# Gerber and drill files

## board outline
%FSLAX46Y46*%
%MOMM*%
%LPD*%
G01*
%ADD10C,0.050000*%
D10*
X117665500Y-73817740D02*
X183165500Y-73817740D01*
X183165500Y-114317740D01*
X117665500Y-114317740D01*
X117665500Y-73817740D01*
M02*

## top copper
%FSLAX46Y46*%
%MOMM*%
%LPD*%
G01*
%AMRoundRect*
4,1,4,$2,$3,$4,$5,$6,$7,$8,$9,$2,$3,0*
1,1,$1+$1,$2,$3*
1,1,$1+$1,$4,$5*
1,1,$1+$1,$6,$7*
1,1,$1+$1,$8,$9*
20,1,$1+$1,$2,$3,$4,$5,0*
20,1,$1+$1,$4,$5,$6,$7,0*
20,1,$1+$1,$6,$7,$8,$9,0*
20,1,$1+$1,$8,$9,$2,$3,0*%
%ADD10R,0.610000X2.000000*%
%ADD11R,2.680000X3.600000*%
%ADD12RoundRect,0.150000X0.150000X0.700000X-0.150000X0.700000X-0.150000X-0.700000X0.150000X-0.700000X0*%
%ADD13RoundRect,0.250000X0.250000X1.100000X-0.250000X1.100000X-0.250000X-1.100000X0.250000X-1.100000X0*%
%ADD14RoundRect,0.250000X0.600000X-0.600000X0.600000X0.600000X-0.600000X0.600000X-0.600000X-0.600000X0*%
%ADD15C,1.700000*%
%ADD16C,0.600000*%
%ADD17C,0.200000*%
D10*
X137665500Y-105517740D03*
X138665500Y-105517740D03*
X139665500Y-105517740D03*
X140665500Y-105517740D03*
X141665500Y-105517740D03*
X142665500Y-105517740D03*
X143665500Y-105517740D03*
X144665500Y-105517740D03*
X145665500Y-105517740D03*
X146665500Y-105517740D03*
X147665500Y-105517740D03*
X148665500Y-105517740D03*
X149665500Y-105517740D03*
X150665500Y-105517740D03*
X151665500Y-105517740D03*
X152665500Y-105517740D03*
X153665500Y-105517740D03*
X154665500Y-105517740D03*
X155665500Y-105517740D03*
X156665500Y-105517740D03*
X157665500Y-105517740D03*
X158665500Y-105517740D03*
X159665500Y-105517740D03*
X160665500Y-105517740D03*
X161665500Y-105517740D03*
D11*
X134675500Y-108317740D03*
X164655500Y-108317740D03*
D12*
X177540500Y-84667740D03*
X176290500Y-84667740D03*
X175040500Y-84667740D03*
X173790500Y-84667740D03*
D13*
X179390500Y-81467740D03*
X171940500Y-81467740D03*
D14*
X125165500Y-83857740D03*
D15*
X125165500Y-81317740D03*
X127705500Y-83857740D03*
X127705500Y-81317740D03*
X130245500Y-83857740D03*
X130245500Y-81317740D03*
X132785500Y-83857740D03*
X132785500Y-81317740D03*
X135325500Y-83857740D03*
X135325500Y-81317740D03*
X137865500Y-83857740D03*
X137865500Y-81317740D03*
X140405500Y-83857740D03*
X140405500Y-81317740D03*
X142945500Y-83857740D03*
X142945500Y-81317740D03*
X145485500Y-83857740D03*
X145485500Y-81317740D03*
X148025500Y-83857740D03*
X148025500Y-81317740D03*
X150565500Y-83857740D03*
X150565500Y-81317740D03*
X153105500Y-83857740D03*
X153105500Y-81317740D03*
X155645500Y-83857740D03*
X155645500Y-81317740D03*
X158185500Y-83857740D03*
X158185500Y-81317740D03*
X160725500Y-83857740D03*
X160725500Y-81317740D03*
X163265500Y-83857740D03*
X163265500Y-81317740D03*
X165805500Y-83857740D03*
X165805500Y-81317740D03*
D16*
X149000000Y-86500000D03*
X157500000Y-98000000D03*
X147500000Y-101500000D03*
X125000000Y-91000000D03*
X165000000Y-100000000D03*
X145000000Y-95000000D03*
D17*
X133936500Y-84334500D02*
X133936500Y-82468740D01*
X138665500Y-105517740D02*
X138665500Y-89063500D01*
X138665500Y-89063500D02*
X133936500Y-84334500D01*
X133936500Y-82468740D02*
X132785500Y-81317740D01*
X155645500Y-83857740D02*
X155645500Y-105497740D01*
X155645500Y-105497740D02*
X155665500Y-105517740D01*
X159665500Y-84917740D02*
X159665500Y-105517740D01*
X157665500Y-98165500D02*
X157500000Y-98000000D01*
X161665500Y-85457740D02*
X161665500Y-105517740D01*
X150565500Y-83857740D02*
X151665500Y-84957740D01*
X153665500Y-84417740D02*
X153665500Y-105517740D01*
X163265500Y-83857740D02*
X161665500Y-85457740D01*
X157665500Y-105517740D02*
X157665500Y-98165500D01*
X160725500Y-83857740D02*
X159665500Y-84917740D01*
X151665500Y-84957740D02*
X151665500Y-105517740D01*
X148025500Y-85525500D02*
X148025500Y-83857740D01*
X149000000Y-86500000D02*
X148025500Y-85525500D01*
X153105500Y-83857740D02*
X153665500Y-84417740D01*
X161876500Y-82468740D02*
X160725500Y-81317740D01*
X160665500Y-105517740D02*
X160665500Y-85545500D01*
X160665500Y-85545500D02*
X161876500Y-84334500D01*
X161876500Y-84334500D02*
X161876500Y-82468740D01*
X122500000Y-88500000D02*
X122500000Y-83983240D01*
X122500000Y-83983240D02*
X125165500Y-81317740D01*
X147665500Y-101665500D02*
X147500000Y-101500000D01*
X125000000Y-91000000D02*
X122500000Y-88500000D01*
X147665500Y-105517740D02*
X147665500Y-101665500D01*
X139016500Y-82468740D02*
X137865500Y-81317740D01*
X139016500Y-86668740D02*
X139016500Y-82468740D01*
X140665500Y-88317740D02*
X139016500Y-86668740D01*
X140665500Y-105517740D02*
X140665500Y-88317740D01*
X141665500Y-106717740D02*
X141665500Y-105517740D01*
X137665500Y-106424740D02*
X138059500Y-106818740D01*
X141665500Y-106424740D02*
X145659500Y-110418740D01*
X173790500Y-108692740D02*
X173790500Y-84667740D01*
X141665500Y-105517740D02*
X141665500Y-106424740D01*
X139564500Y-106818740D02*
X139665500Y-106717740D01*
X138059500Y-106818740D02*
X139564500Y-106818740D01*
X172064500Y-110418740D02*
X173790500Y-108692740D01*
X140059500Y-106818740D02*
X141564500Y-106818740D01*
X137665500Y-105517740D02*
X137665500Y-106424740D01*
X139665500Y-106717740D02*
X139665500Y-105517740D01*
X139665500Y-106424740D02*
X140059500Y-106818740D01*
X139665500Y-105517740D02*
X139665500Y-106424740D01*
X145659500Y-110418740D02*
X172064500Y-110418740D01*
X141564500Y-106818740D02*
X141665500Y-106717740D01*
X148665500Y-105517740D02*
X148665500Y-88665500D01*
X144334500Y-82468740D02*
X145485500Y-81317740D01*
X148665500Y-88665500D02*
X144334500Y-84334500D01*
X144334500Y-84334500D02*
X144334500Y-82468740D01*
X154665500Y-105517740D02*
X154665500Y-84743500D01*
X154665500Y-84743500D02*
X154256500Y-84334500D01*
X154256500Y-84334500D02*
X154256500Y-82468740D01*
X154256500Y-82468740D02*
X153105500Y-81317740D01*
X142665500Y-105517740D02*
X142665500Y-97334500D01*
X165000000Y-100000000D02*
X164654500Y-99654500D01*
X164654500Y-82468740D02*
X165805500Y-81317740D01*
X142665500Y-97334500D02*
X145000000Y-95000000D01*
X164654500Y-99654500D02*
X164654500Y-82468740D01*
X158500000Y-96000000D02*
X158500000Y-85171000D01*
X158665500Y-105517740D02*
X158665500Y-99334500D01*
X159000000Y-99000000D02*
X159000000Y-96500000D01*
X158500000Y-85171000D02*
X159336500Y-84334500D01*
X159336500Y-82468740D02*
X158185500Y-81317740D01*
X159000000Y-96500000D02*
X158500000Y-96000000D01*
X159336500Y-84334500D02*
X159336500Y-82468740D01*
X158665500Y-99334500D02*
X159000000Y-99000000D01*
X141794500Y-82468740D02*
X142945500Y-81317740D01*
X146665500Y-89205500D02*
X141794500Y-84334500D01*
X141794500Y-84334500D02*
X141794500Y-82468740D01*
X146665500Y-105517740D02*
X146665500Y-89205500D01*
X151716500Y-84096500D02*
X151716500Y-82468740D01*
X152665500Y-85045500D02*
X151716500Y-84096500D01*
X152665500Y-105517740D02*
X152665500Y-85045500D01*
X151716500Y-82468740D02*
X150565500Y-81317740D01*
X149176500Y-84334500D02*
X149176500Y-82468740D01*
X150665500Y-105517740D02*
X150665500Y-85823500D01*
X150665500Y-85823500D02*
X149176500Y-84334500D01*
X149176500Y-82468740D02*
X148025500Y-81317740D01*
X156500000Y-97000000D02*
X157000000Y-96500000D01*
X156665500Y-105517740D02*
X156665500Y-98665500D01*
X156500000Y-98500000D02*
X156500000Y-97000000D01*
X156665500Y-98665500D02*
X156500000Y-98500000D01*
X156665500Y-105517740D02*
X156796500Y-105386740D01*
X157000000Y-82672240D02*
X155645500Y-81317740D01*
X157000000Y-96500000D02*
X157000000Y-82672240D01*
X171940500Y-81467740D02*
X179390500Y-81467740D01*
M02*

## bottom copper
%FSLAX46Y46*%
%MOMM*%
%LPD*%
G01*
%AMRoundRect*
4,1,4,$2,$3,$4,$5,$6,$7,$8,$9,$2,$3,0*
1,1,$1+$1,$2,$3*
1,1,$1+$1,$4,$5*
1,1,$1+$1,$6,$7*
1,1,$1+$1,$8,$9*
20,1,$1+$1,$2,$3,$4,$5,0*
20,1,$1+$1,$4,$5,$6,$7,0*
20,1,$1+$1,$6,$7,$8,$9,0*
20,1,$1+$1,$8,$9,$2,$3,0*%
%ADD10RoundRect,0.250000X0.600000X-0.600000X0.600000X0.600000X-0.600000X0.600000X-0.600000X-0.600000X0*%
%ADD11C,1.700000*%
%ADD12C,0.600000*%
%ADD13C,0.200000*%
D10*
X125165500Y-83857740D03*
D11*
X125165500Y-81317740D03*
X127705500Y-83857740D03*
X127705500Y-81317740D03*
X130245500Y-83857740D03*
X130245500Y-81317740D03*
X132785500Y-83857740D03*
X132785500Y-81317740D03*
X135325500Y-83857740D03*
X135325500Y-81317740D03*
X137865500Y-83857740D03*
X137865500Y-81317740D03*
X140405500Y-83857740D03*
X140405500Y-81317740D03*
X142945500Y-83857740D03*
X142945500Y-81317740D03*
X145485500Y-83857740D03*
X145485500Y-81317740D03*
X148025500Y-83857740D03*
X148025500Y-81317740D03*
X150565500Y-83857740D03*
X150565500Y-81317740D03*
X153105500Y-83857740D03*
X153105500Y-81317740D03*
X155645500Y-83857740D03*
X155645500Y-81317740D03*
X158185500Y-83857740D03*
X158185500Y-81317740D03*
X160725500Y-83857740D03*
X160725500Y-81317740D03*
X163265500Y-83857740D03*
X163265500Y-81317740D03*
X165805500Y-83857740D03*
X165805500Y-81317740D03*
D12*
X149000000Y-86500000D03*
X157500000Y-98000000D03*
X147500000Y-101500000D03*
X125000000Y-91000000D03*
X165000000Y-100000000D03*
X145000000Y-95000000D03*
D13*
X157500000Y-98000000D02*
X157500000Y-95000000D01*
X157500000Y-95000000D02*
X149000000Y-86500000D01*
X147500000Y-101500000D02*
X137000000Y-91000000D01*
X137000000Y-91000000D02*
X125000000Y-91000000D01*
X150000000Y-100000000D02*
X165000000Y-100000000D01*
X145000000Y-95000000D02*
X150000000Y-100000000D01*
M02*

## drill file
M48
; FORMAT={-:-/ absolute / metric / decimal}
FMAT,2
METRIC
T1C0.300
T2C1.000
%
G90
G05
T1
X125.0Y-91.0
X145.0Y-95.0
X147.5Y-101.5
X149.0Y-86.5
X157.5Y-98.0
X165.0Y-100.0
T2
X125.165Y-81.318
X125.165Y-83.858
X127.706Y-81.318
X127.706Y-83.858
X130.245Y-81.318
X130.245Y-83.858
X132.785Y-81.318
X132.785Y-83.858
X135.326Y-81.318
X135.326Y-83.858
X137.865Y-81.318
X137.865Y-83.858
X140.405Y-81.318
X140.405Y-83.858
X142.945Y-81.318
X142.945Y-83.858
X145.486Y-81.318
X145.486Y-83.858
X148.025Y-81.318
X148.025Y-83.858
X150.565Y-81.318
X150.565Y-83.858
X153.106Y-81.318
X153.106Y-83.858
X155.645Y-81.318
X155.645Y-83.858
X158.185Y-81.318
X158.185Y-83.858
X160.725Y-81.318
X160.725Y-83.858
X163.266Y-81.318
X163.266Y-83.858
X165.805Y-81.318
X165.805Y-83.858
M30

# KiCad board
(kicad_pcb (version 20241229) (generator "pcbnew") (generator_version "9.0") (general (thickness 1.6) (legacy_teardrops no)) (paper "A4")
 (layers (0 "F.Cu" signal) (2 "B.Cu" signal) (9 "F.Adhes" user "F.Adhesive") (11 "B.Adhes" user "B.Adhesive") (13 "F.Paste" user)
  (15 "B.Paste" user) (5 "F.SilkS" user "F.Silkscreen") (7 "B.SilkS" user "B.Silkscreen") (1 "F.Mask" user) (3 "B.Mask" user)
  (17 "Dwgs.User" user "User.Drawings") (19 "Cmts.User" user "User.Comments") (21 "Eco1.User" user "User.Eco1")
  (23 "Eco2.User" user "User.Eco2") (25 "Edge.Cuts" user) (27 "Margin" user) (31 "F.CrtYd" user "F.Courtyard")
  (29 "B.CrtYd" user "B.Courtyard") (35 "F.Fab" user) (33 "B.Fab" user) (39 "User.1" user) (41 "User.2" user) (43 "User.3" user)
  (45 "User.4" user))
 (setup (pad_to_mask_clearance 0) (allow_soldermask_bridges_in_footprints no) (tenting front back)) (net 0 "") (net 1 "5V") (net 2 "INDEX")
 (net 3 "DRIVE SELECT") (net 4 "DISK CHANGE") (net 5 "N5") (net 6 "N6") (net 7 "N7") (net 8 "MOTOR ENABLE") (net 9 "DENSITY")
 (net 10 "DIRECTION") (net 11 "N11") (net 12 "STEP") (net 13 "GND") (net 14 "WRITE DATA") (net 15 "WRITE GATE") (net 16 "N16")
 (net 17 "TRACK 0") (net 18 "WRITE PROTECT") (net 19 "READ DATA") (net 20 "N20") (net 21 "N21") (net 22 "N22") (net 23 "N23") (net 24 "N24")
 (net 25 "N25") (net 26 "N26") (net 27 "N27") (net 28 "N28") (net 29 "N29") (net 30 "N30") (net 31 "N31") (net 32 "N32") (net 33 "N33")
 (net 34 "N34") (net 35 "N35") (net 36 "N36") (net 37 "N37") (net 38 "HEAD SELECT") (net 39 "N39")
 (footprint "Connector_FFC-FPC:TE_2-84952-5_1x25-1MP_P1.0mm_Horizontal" (layer "F.Cu") (at 149.6655 107.31774)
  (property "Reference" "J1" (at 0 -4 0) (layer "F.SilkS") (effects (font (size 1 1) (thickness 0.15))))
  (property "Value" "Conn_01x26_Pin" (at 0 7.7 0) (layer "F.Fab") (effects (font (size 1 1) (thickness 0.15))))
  (pad "1" smd rect (at -12 -1.8) (size 0.61 2) (layers "F.Cu" "F.Mask" "F.Paste") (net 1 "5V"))
  (pad "2" smd rect (at -11 -1.8) (size 0.61 2) (layers "F.Cu" "F.Mask" "F.Paste") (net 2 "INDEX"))
  (pad "3" smd rect (at -10 -1.8) (size 0.61 2) (layers "F.Cu" "F.Mask" "F.Paste") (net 1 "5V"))
  (pad "4" smd rect (at -9 -1.8) (size 0.61 2) (layers "F.Cu" "F.Mask" "F.Paste") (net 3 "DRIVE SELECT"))
  (pad "5" smd rect (at -8 -1.8) (size 0.61 2) (layers "F.Cu" "F.Mask" "F.Paste") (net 1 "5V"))
  (pad "6" smd rect (at -7 -1.8) (size 0.61 2) (layers "F.Cu" "F.Mask" "F.Paste") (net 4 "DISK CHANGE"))
  (pad "7" smd rect (at -6 -1.8) (size 0.61 2) (layers "F.Cu" "F.Mask" "F.Paste") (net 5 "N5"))
  (pad "8" smd rect (at -5 -1.8) (size 0.61 2) (layers "F.Cu" "F.Mask" "F.Paste") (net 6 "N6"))
  (pad "9" smd rect (at -4 -1.8) (size 0.61 2) (layers "F.Cu" "F.Mask" "F.Paste") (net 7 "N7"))
  (pad "10" smd rect (at -3 -1.8) (size 0.61 2) (layers "F.Cu" "F.Mask" "F.Paste") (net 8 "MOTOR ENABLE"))
  (pad "11" smd rect (at -2 -1.8) (size 0.61 2) (layers "F.Cu" "F.Mask" "F.Paste") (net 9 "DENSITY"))
  (pad "12" smd rect (at -1 -1.8) (size 0.61 2) (layers "F.Cu" "F.Mask" "F.Paste") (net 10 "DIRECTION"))
  (pad "13" smd rect (at 0 -1.8) (size 0.61 2) (layers "F.Cu" "F.Mask" "F.Paste") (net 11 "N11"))
  (pad "14" smd rect (at 1 -1.8) (size 0.61 2) (layers "F.Cu" "F.Mask" "F.Paste") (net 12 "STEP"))
  (pad "15" smd rect (at 2 -1.8) (size 0.61 2) (layers "F.Cu" "F.Mask" "F.Paste") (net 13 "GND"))
  (pad "16" smd rect (at 3 -1.8) (size 0.61 2) (layers "F.Cu" "F.Mask" "F.Paste") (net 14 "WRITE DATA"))
  (pad "17" smd rect (at 4 -1.8) (size 0.61 2) (layers "F.Cu" "F.Mask" "F.Paste") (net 13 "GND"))
  (pad "18" smd rect (at 5 -1.8) (size 0.61 2) (layers "F.Cu" "F.Mask" "F.Paste") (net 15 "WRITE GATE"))
  (pad "19" smd rect (at 6 -1.8) (size 0.61 2) (layers "F.Cu" "F.Mask" "F.Paste") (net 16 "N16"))
  (pad "20" smd rect (at 7 -1.8) (size 0.61 2) (layers "F.Cu" "F.Mask" "F.Paste") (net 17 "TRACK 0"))
  (pad "21" smd rect (at 8 -1.8) (size 0.61 2) (layers "F.Cu" "F.Mask" "F.Paste") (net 13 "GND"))
  (pad "22" smd rect (at 9 -1.8) (size 0.61 2) (layers "F.Cu" "F.Mask" "F.Paste") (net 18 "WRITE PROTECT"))
  (pad "23" smd rect (at 10 -1.8) (size 0.61 2) (layers "F.Cu" "F.Mask" "F.Paste") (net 13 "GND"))
  (pad "24" smd rect (at 11 -1.8) (size 0.61 2) (layers "F.Cu" "F.Mask" "F.Paste") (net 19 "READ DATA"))
  (pad "25" smd rect (at 12 -1.8) (size 0.61 2) (layers "F.Cu" "F.Mask" "F.Paste") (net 13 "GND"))
  (pad "MP" smd rect (at -14.99 1) (size 2.68 3.6) (layers "F.Cu" "F.Mask" "F.Paste"))
  (pad "MP" smd rect (at 14.99 1) (size 2.68 3.6) (layers "F.Cu" "F.Mask" "F.Paste")))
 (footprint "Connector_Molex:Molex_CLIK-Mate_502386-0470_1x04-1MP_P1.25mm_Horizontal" (layer "F.Cu") (at 175.6655 82.81774 180)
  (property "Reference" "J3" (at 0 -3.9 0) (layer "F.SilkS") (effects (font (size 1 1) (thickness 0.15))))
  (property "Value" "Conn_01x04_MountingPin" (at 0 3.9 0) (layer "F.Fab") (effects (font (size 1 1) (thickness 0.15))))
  (pad "1" smd roundrect (at -1.875 -1.85 180) (size 0.6 1.7) (layers "F.Cu" "F.Mask" "F.Paste") (roundrect_rratio 0.25) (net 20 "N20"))
  (pad "2" smd roundrect (at -0.625 -1.85 180) (size 0.6 1.7) (layers "F.Cu" "F.Mask" "F.Paste") (roundrect_rratio 0.25) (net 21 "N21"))
  (pad "3" smd roundrect (at 0.625 -1.85 180) (size 0.6 1.7) (layers "F.Cu" "F.Mask" "F.Paste") (roundrect_rratio 0.25) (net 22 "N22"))
  (pad "4" smd roundrect (at 1.875 -1.85 180) (size 0.6 1.7) (layers "F.Cu" "F.Mask" "F.Paste") (roundrect_rratio 0.25) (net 1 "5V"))
  (pad "MP" smd roundrect (at -3.725 1.35 180) (size 1 2.7) (layers "F.Cu" "F.Mask" "F.Paste") (roundrect_rratio 0.25) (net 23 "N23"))
  (pad "MP" smd roundrect (at 3.725 1.35 180) (size 1 2.7) (layers "F.Cu" "F.Mask" "F.Paste") (roundrect_rratio 0.25) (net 23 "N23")))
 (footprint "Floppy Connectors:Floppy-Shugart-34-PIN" (layer "F.Cu") (at 125.1655 83.85774 90)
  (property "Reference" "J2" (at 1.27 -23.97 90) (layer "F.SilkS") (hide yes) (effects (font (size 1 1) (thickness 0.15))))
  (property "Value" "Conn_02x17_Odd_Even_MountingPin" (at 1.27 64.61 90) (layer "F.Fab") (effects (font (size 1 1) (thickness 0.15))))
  (pad "1" thru_hole roundrect (at 0 0 90) (size 1.7 1.7) (drill 1) (layers "*.Cu" "*.Mask") (remove_unused_layers no)
   (roundrect_rratio 0.147059) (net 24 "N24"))
  (pad "2" thru_hole circle (at 2.54 0 90) (size 1.7 1.7) (drill 1) (layers "*.Cu" "*.Mask") (remove_unused_layers no) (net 9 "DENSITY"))
  (pad "3" thru_hole circle (at 0 2.54 90) (size 1.7 1.7) (drill 1) (layers "*.Cu" "*.Mask") (remove_unused_layers no) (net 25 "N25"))
  (pad "4" thru_hole circle (at 2.54 2.54 90) (size 1.7 1.7) (drill 1) (layers "*.Cu" "*.Mask") (remove_unused_layers no) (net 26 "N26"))
  (pad "5" thru_hole circle (at 0 5.08 90) (size 1.7 1.7) (drill 1) (layers "*.Cu" "*.Mask") (remove_unused_layers no) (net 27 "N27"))
  (pad "6" thru_hole circle (at 2.54 5.08 90) (size 1.7 1.7) (drill 1) (layers "*.Cu" "*.Mask") (remove_unused_layers no) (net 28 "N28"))
  (pad "7" thru_hole circle (at 0 7.62 90) (size 1.7 1.7) (drill 1) (layers "*.Cu" "*.Mask") (remove_unused_layers no) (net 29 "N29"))
  (pad "8" thru_hole circle (at 2.54 7.62 90) (size 1.7 1.7) (drill 1) (layers "*.Cu" "*.Mask") (remove_unused_layers no) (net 2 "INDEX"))
  (pad "9" thru_hole circle (at 0 10.16 90) (size 1.7 1.7) (drill 1) (layers "*.Cu" "*.Mask") (remove_unused_layers no) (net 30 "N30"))
  (pad "10" thru_hole circle (at 2.54 10.16 90) (size 1.7 1.7) (drill 1) (layers "*.Cu" "*.Mask") (remove_unused_layers no) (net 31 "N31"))
  (pad "11" thru_hole circle (at 0 12.7 90) (size 1.7 1.7) (drill 1) (layers "*.Cu" "*.Mask") (remove_unused_layers no) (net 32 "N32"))
  (pad "12" thru_hole circle (at 2.54 12.7 90) (size 1.7 1.7) (drill 1) (layers "*.Cu" "*.Mask") (remove_unused_layers no)
   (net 3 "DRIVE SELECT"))
  (pad "13" thru_hole circle (at 0 15.24 90) (size 1.7 1.7) (drill 1) (layers "*.Cu" "*.Mask") (remove_unused_layers no) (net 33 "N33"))
  (pad "14" thru_hole circle (at 2.54 15.24 90) (size 1.7 1.7) (drill 1) (layers "*.Cu" "*.Mask") (remove_unused_layers no) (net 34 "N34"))
  (pad "15" thru_hole circle (at 0 17.78 90) (size 1.7 1.7) (drill 1) (layers "*.Cu" "*.Mask") (remove_unused_layers no) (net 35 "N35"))
  (pad "16" thru_hole circle (at 2.54 17.78 90) (size 1.7 1.7) (drill 1) (layers "*.Cu" "*.Mask") (remove_unused_layers no)
   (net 8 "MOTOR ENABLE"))
  (pad "17" thru_hole circle (at 0 20.32 90) (size 1.7 1.7) (drill 1) (layers "*.Cu" "*.Mask") (remove_unused_layers no) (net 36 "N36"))
  (pad "18" thru_hole circle (at 2.54 20.32 90) (size 1.7 1.7) (drill 1) (layers "*.Cu" "*.Mask") (remove_unused_layers no)
   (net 10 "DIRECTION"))
  (pad "19" thru_hole circle (at 0 22.86 90) (size 1.7 1.7) (drill 1) (layers "*.Cu" "*.Mask") (remove_unused_layers no) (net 13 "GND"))
  (pad "20" thru_hole circle (at 2.54 22.86 90) (size 1.7 1.7) (drill 1) (layers "*.Cu" "*.Mask") (remove_unused_layers no) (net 12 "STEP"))
  (pad "21" thru_hole circle (at 0 25.4 90) (size 1.7 1.7) (drill 1) (layers "*.Cu" "*.Mask") (remove_unused_layers no) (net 13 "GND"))
  (pad "22" thru_hole circle (at 2.54 25.4 90) (size 1.7 1.7) (drill 1) (layers "*.Cu" "*.Mask") (remove_unused_layers no)
   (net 14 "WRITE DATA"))
  (pad "23" thru_hole circle (at 0 27.94 90) (size 1.7 1.7) (drill 1) (layers "*.Cu" "*.Mask") (remove_unused_layers no) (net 13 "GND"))
  (pad "24" thru_hole circle (at 2.54 27.94 90) (size 1.7 1.7) (drill 1) (layers "*.Cu" "*.Mask") (remove_unused_layers no)
   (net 15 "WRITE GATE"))
  (pad "25" thru_hole circle (at 0 30.48 90) (size 1.7 1.7) (drill 1) (layers "*.Cu" "*.Mask") (remove_unused_layers no) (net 16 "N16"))
  (pad "26" thru_hole circle (at 2.54 30.48 90) (size 1.7 1.7) (drill 1) (layers "*.Cu" "*.Mask") (remove_unused_layers no)
   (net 17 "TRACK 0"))
  (pad "27" thru_hole circle (at 0 33.02 90) (size 1.7 1.7) (drill 1) (layers "*.Cu" "*.Mask") (remove_unused_layers no) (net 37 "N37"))
  (pad "28" thru_hole circle (at 2.54 33.02 90) (size 1.7 1.7) (drill 1) (layers "*.Cu" "*.Mask") (remove_unused_layers no)
   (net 18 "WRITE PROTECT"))
  (pad "29" thru_hole circle (at 0 35.56 90) (size 1.7 1.7) (drill 1) (layers "*.Cu" "*.Mask") (remove_unused_layers no) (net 13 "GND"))
  (pad "30" thru_hole circle (at 2.54 35.56 90) (size 1.7 1.7) (drill 1) (layers "*.Cu" "*.Mask") (remove_unused_layers no)
   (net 19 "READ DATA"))
  (pad "31" thru_hole circle (at 0 38.1 90) (size 1.7 1.7) (drill 1) (layers "*.Cu" "*.Mask") (remove_unused_layers no) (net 13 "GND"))
  (pad "32" thru_hole circle (at 2.54 38.1 90) (size 1.7 1.7) (drill 1) (layers "*.Cu" "*.Mask") (remove_unused_layers no)
   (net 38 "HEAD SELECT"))
  (pad "33" thru_hole circle (at 0 40.64 90) (size 1.7 1.7) (drill 1) (layers "*.Cu" "*.Mask") (remove_unused_layers no) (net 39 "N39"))
  (pad "34" thru_hole circle (at 2.54 40.64 90) (size 1.7 1.7) (drill 1) (layers "*.Cu" "*.Mask") (remove_unused_layers no)
   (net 4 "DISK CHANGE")))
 (gr_rect (start 117.6655 73.81774) (end 183.1655 114.31774) (stroke (width 0.05) (type default)) (fill no) (layer "Edge.Cuts"))
 (segment (start 133.9365 84.3345) (end 133.9365 82.46874) (width 0.2) (layer "F.Cu") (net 2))
 (segment (start 138.6655 105.51774) (end 138.6655 89.0635) (width 0.2) (layer "F.Cu") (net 2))
 (segment (start 138.6655 89.0635) (end 133.9365 84.3345) (width 0.2) (layer "F.Cu") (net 2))
 (segment (start 133.9365 82.46874) (end 132.7855 81.31774) (width 0.2) (layer "F.Cu") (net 2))
 (segment (start 155.6455 83.85774) (end 155.6455 105.49774) (width 0.2) (layer "F.Cu") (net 16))
 (segment (start 155.6455 105.49774) (end 155.6655 105.51774) (width 0.2) (layer "F.Cu") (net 16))
 (segment (start 159.6655 84.91774) (end 159.6655 105.51774) (width 0.2) (layer "F.Cu") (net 13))
 (segment (start 157.6655 98.1655) (end 157.5 98) (width 0.2) (layer "F.Cu") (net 13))
 (segment (start 161.6655 85.45774) (end 161.6655 105.51774) (width 0.2) (layer "F.Cu") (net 13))
 (segment (start 150.5655 83.85774) (end 151.6655 84.95774) (width 0.2) (layer "F.Cu") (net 13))
 (segment (start 153.6655 84.41774) (end 153.6655 105.51774) (width 0.2) (layer "F.Cu") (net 13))
 (segment (start 163.2655 83.85774) (end 161.6655 85.45774) (width 0.2) (layer "F.Cu") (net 13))
 (segment (start 157.6655 105.51774) (end 157.6655 98.1655) (width 0.2) (layer "F.Cu") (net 13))
 (segment (start 160.7255 83.85774) (end 159.6655 84.91774) (width 0.2) (layer "F.Cu") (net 13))
 (segment (start 151.6655 84.95774) (end 151.6655 105.51774) (width 0.2) (layer "F.Cu") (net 13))
 (segment (start 148.0255 85.5255) (end 148.0255 83.85774) (width 0.2) (layer "F.Cu") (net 13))
 (segment (start 149 86.5) (end 148.0255 85.5255) (width 0.2) (layer "F.Cu") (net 13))
 (segment (start 153.1055 83.85774) (end 153.6655 84.41774) (width 0.2) (layer "F.Cu") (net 13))
 (via (at 149 86.5) (size 0.6) (drill 0.3) (layers "F.Cu" "B.Cu") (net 13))
 (via (at 157.5 98) (size 0.6) (drill 0.3) (layers "F.Cu" "B.Cu") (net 13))
 (segment (start 157.5 98) (end 157.5 95) (width 0.2) (layer "B.Cu") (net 13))
 (segment (start 157.5 95) (end 149 86.5) (width 0.2) (layer "B.Cu") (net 13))
 (segment (start 161.8765 82.46874) (end 160.7255 81.31774) (width 0.2) (layer "F.Cu") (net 19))
 (segment (start 160.6655 105.51774) (end 160.6655 85.5455) (width 0.2) (layer "F.Cu") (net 19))
 (segment (start 160.6655 85.5455) (end 161.8765 84.3345) (width 0.2) (layer "F.Cu") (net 19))
 (segment (start 161.8765 84.3345) (end 161.8765 82.46874) (width 0.2) (layer "F.Cu") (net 19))
 (segment (start 122.5 88.5) (end 122.5 83.98324) (width 0.2) (layer "F.Cu") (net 9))
 (segment (start 122.5 83.98324) (end 125.1655 81.31774) (width 0.2) (layer "F.Cu") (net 9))
 (segment (start 147.6655 101.6655) (end 147.5 101.5) (width 0.2) (layer "F.Cu") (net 9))
 (segment (start 125 91) (end 122.5 88.5) (width 0.2) (layer "F.Cu") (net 9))
 (segment (start 147.6655 105.51774) (end 147.6655 101.6655) (width 0.2) (layer "F.Cu") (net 9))
 (via (at 147.5 101.5) (size 0.6) (drill 0.3) (layers "F.Cu" "B.Cu") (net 9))
 (via (at 125 91) (size 0.6) (drill 0.3) (layers "F.Cu" "B.Cu") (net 9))
 (segment (start 147.5 101.5) (end 137 91) (width 0.2) (layer "B.Cu") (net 9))
 (segment (start 137 91) (end 125 91) (width 0.2) (layer "B.Cu") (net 9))
 (segment (start 139.0165 82.46874) (end 137.8655 81.31774) (width 0.2) (layer "F.Cu") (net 3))
 (segment (start 139.0165 86.66874) (end 139.0165 82.46874) (width 0.2) (layer "F.Cu") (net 3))
 (segment (start 140.6655 88.31774) (end 139.0165 86.66874) (width 0.2) (layer "F.Cu") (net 3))
 (segment (start 140.6655 105.51774) (end 140.6655 88.31774) (width 0.2) (layer "F.Cu") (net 3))
 (segment (start 141.6655 106.71774) (end 141.6655 105.51774) (width 0.2) (layer "F.Cu") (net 1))
 (segment (start 137.6655 106.42474) (end 138.0595 106.81874) (width 0.2) (layer "F.Cu") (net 1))
 (segment (start 141.6655 106.42474) (end 145.6595 110.41874) (width 0.2) (layer "F.Cu") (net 1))
 (segment (start 173.7905 108.69274) (end 173.7905 84.66774) (width 0.2) (layer "F.Cu") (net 1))
 (segment (start 141.6655 105.51774) (end 141.6655 106.42474) (width 0.2) (layer "F.Cu") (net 1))
 (segment (start 139.5645 106.81874) (end 139.6655 106.71774) (width 0.2) (layer "F.Cu") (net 1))
 (segment (start 138.0595 106.81874) (end 139.5645 106.81874) (width 0.2) (layer "F.Cu") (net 1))
 (segment (start 172.0645 110.41874) (end 173.7905 108.69274) (width 0.2) (layer "F.Cu") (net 1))
 (segment (start 140.0595 106.81874) (end 141.5645 106.81874) (width 0.2) (layer "F.Cu") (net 1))
 (segment (start 137.6655 105.51774) (end 137.6655 106.42474) (width 0.2) (layer "F.Cu") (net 1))
 (segment (start 139.6655 106.71774) (end 139.6655 105.51774) (width 0.2) (layer "F.Cu") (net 1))
 (segment (start 139.6655 106.42474) (end 140.0595 106.81874) (width 0.2) (layer "F.Cu") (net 1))
 (segment (start 139.6655 105.51774) (end 139.6655 106.42474) (width 0.2) (layer "F.Cu") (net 1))
 (segment (start 145.6595 110.41874) (end 172.0645 110.41874) (width 0.2) (layer "F.Cu") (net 1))
 (segment (start 141.5645 106.81874) (end 141.6655 106.71774) (width 0.2) (layer "F.Cu") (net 1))
 (segment (start 148.6655 105.51774) (end 148.6655 88.6655) (width 0.2) (layer "F.Cu") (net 10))
 (segment (start 144.3345 82.46874) (end 145.4855 81.31774) (width 0.2) (layer "F.Cu") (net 10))
 (segment (start 148.6655 88.6655) (end 144.3345 84.3345) (width 0.2) (layer "F.Cu") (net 10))
 (segment (start 144.3345 84.3345) (end 144.3345 82.46874) (width 0.2) (layer "F.Cu") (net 10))
 (segment (start 154.6655 105.51774) (end 154.6655 84.7435) (width 0.2) (layer "F.Cu") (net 15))
 (segment (start 154.6655 84.7435) (end 154.2565 84.3345) (width 0.2) (layer "F.Cu") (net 15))
 (segment (start 154.2565 84.3345) (end 154.2565 82.46874) (width 0.2) (layer "F.Cu") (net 15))
 (segment (start 154.2565 82.46874) (end 153.1055 81.31774) (width 0.2) (layer "F.Cu") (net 15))
 (segment (start 142.6655 105.51774) (end 142.6655 97.3345) (width 0.2) (layer "F.Cu") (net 4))
 (segment (start 165 100) (end 164.6545 99.6545) (width 0.2) (layer "F.Cu") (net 4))
 (segment (start 164.6545 82.46874) (end 165.8055 81.31774) (width 0.2) (layer "F.Cu") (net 4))
 (segment (start 142.6655 97.3345) (end 145 95) (width 0.2) (layer "F.Cu") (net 4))
 (segment (start 164.6545 99.6545) (end 164.6545 82.46874) (width 0.2) (layer "F.Cu") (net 4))
 (via (at 165 100) (size 0.6) (drill 0.3) (layers "F.Cu" "B.Cu") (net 4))
 (via (at 145 95) (size 0.6) (drill 0.3) (layers "F.Cu" "B.Cu") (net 4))
 (segment (start 150 100) (end 165 100) (width 0.2) (layer "B.Cu") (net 4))
 (segment (start 145 95) (end 150 100) (width 0.2) (layer "B.Cu") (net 4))
 (segment (start 158.5 96) (end 158.5 85.171) (width 0.2) (layer "F.Cu") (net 18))
 (segment (start 158.6655 105.51774) (end 158.6655 99.3345) (width 0.2) (layer "F.Cu") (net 18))
 (segment (start 159 99) (end 159 96.5) (width 0.2) (layer "F.Cu") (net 18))
 (segment (start 158.5 85.171) (end 159.3365 84.3345) (width 0.2) (layer "F.Cu") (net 18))
 (segment (start 159.3365 82.46874) (end 158.1855 81.31774) (width 0.2) (layer "F.Cu") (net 18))
 (segment (start 159 96.5) (end 158.5 96) (width 0.2) (layer "F.Cu") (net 18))
 (segment (start 159.3365 84.3345) (end 159.3365 82.46874) (width 0.2) (layer "F.Cu") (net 18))
 (segment (start 158.6655 99.3345) (end 159 99) (width 0.2) (layer "F.Cu") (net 18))
 (segment (start 141.7945 82.46874) (end 142.9455 81.31774) (width 0.2) (layer "F.Cu") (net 8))
 (segment (start 146.6655 89.2055) (end 141.7945 84.3345) (width 0.2) (layer "F.Cu") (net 8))
 (segment (start 141.7945 84.3345) (end 141.7945 82.46874) (width 0.2) (layer "F.Cu") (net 8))
 (segment (start 146.6655 105.51774) (end 146.6655 89.2055) (width 0.2) (layer "F.Cu") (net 8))
 (segment (start 151.7165 84.0965) (end 151.7165 82.46874) (width 0.2) (layer "F.Cu") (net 14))
 (segment (start 152.6655 85.0455) (end 151.7165 84.0965) (width 0.2) (layer "F.Cu") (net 14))
 (segment (start 152.6655 105.51774) (end 152.6655 85.0455) (width 0.2) (layer "F.Cu") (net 14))
 (segment (start 151.7165 82.46874) (end 150.5655 81.31774) (width 0.2) (layer "F.Cu") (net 14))
 (segment (start 149.1765 84.3345) (end 149.1765 82.46874) (width 0.2) (layer "F.Cu") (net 12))
 (segment (start 150.6655 105.51774) (end 150.6655 85.8235) (width 0.2) (layer "F.Cu") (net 12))
 (segment (start 150.6655 85.8235) (end 149.1765 84.3345) (width 0.2) (layer "F.Cu") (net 12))
 (segment (start 149.1765 82.46874) (end 148.0255 81.31774) (width 0.2) (layer "F.Cu") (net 12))
 (segment (start 156.5 97) (end 157 96.5) (width 0.2) (layer "F.Cu") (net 17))
 (segment (start 156.6655 105.51774) (end 156.6655 98.6655) (width 0.2) (layer "F.Cu") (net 17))
 (segment (start 156.5 98.5) (end 156.5 97) (width 0.2) (layer "F.Cu") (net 17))
 (segment (start 156.6655 98.6655) (end 156.5 98.5) (width 0.2) (layer "F.Cu") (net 17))
 (segment (start 156.6655 105.51774) (end 156.7965 105.38674) (width 0.2) (layer "F.Cu") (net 17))
 (segment (start 157 82.67224) (end 155.6455 81.31774) (width 0.2) (layer "F.Cu") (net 17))
 (segment (start 157 96.5) (end 157 82.67224) (width 0.2) (layer "F.Cu") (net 17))
 (segment (start 171.9405 81.46774) (end 179.3905 81.46774) (width 0.2) (layer "F.Cu") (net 23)))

